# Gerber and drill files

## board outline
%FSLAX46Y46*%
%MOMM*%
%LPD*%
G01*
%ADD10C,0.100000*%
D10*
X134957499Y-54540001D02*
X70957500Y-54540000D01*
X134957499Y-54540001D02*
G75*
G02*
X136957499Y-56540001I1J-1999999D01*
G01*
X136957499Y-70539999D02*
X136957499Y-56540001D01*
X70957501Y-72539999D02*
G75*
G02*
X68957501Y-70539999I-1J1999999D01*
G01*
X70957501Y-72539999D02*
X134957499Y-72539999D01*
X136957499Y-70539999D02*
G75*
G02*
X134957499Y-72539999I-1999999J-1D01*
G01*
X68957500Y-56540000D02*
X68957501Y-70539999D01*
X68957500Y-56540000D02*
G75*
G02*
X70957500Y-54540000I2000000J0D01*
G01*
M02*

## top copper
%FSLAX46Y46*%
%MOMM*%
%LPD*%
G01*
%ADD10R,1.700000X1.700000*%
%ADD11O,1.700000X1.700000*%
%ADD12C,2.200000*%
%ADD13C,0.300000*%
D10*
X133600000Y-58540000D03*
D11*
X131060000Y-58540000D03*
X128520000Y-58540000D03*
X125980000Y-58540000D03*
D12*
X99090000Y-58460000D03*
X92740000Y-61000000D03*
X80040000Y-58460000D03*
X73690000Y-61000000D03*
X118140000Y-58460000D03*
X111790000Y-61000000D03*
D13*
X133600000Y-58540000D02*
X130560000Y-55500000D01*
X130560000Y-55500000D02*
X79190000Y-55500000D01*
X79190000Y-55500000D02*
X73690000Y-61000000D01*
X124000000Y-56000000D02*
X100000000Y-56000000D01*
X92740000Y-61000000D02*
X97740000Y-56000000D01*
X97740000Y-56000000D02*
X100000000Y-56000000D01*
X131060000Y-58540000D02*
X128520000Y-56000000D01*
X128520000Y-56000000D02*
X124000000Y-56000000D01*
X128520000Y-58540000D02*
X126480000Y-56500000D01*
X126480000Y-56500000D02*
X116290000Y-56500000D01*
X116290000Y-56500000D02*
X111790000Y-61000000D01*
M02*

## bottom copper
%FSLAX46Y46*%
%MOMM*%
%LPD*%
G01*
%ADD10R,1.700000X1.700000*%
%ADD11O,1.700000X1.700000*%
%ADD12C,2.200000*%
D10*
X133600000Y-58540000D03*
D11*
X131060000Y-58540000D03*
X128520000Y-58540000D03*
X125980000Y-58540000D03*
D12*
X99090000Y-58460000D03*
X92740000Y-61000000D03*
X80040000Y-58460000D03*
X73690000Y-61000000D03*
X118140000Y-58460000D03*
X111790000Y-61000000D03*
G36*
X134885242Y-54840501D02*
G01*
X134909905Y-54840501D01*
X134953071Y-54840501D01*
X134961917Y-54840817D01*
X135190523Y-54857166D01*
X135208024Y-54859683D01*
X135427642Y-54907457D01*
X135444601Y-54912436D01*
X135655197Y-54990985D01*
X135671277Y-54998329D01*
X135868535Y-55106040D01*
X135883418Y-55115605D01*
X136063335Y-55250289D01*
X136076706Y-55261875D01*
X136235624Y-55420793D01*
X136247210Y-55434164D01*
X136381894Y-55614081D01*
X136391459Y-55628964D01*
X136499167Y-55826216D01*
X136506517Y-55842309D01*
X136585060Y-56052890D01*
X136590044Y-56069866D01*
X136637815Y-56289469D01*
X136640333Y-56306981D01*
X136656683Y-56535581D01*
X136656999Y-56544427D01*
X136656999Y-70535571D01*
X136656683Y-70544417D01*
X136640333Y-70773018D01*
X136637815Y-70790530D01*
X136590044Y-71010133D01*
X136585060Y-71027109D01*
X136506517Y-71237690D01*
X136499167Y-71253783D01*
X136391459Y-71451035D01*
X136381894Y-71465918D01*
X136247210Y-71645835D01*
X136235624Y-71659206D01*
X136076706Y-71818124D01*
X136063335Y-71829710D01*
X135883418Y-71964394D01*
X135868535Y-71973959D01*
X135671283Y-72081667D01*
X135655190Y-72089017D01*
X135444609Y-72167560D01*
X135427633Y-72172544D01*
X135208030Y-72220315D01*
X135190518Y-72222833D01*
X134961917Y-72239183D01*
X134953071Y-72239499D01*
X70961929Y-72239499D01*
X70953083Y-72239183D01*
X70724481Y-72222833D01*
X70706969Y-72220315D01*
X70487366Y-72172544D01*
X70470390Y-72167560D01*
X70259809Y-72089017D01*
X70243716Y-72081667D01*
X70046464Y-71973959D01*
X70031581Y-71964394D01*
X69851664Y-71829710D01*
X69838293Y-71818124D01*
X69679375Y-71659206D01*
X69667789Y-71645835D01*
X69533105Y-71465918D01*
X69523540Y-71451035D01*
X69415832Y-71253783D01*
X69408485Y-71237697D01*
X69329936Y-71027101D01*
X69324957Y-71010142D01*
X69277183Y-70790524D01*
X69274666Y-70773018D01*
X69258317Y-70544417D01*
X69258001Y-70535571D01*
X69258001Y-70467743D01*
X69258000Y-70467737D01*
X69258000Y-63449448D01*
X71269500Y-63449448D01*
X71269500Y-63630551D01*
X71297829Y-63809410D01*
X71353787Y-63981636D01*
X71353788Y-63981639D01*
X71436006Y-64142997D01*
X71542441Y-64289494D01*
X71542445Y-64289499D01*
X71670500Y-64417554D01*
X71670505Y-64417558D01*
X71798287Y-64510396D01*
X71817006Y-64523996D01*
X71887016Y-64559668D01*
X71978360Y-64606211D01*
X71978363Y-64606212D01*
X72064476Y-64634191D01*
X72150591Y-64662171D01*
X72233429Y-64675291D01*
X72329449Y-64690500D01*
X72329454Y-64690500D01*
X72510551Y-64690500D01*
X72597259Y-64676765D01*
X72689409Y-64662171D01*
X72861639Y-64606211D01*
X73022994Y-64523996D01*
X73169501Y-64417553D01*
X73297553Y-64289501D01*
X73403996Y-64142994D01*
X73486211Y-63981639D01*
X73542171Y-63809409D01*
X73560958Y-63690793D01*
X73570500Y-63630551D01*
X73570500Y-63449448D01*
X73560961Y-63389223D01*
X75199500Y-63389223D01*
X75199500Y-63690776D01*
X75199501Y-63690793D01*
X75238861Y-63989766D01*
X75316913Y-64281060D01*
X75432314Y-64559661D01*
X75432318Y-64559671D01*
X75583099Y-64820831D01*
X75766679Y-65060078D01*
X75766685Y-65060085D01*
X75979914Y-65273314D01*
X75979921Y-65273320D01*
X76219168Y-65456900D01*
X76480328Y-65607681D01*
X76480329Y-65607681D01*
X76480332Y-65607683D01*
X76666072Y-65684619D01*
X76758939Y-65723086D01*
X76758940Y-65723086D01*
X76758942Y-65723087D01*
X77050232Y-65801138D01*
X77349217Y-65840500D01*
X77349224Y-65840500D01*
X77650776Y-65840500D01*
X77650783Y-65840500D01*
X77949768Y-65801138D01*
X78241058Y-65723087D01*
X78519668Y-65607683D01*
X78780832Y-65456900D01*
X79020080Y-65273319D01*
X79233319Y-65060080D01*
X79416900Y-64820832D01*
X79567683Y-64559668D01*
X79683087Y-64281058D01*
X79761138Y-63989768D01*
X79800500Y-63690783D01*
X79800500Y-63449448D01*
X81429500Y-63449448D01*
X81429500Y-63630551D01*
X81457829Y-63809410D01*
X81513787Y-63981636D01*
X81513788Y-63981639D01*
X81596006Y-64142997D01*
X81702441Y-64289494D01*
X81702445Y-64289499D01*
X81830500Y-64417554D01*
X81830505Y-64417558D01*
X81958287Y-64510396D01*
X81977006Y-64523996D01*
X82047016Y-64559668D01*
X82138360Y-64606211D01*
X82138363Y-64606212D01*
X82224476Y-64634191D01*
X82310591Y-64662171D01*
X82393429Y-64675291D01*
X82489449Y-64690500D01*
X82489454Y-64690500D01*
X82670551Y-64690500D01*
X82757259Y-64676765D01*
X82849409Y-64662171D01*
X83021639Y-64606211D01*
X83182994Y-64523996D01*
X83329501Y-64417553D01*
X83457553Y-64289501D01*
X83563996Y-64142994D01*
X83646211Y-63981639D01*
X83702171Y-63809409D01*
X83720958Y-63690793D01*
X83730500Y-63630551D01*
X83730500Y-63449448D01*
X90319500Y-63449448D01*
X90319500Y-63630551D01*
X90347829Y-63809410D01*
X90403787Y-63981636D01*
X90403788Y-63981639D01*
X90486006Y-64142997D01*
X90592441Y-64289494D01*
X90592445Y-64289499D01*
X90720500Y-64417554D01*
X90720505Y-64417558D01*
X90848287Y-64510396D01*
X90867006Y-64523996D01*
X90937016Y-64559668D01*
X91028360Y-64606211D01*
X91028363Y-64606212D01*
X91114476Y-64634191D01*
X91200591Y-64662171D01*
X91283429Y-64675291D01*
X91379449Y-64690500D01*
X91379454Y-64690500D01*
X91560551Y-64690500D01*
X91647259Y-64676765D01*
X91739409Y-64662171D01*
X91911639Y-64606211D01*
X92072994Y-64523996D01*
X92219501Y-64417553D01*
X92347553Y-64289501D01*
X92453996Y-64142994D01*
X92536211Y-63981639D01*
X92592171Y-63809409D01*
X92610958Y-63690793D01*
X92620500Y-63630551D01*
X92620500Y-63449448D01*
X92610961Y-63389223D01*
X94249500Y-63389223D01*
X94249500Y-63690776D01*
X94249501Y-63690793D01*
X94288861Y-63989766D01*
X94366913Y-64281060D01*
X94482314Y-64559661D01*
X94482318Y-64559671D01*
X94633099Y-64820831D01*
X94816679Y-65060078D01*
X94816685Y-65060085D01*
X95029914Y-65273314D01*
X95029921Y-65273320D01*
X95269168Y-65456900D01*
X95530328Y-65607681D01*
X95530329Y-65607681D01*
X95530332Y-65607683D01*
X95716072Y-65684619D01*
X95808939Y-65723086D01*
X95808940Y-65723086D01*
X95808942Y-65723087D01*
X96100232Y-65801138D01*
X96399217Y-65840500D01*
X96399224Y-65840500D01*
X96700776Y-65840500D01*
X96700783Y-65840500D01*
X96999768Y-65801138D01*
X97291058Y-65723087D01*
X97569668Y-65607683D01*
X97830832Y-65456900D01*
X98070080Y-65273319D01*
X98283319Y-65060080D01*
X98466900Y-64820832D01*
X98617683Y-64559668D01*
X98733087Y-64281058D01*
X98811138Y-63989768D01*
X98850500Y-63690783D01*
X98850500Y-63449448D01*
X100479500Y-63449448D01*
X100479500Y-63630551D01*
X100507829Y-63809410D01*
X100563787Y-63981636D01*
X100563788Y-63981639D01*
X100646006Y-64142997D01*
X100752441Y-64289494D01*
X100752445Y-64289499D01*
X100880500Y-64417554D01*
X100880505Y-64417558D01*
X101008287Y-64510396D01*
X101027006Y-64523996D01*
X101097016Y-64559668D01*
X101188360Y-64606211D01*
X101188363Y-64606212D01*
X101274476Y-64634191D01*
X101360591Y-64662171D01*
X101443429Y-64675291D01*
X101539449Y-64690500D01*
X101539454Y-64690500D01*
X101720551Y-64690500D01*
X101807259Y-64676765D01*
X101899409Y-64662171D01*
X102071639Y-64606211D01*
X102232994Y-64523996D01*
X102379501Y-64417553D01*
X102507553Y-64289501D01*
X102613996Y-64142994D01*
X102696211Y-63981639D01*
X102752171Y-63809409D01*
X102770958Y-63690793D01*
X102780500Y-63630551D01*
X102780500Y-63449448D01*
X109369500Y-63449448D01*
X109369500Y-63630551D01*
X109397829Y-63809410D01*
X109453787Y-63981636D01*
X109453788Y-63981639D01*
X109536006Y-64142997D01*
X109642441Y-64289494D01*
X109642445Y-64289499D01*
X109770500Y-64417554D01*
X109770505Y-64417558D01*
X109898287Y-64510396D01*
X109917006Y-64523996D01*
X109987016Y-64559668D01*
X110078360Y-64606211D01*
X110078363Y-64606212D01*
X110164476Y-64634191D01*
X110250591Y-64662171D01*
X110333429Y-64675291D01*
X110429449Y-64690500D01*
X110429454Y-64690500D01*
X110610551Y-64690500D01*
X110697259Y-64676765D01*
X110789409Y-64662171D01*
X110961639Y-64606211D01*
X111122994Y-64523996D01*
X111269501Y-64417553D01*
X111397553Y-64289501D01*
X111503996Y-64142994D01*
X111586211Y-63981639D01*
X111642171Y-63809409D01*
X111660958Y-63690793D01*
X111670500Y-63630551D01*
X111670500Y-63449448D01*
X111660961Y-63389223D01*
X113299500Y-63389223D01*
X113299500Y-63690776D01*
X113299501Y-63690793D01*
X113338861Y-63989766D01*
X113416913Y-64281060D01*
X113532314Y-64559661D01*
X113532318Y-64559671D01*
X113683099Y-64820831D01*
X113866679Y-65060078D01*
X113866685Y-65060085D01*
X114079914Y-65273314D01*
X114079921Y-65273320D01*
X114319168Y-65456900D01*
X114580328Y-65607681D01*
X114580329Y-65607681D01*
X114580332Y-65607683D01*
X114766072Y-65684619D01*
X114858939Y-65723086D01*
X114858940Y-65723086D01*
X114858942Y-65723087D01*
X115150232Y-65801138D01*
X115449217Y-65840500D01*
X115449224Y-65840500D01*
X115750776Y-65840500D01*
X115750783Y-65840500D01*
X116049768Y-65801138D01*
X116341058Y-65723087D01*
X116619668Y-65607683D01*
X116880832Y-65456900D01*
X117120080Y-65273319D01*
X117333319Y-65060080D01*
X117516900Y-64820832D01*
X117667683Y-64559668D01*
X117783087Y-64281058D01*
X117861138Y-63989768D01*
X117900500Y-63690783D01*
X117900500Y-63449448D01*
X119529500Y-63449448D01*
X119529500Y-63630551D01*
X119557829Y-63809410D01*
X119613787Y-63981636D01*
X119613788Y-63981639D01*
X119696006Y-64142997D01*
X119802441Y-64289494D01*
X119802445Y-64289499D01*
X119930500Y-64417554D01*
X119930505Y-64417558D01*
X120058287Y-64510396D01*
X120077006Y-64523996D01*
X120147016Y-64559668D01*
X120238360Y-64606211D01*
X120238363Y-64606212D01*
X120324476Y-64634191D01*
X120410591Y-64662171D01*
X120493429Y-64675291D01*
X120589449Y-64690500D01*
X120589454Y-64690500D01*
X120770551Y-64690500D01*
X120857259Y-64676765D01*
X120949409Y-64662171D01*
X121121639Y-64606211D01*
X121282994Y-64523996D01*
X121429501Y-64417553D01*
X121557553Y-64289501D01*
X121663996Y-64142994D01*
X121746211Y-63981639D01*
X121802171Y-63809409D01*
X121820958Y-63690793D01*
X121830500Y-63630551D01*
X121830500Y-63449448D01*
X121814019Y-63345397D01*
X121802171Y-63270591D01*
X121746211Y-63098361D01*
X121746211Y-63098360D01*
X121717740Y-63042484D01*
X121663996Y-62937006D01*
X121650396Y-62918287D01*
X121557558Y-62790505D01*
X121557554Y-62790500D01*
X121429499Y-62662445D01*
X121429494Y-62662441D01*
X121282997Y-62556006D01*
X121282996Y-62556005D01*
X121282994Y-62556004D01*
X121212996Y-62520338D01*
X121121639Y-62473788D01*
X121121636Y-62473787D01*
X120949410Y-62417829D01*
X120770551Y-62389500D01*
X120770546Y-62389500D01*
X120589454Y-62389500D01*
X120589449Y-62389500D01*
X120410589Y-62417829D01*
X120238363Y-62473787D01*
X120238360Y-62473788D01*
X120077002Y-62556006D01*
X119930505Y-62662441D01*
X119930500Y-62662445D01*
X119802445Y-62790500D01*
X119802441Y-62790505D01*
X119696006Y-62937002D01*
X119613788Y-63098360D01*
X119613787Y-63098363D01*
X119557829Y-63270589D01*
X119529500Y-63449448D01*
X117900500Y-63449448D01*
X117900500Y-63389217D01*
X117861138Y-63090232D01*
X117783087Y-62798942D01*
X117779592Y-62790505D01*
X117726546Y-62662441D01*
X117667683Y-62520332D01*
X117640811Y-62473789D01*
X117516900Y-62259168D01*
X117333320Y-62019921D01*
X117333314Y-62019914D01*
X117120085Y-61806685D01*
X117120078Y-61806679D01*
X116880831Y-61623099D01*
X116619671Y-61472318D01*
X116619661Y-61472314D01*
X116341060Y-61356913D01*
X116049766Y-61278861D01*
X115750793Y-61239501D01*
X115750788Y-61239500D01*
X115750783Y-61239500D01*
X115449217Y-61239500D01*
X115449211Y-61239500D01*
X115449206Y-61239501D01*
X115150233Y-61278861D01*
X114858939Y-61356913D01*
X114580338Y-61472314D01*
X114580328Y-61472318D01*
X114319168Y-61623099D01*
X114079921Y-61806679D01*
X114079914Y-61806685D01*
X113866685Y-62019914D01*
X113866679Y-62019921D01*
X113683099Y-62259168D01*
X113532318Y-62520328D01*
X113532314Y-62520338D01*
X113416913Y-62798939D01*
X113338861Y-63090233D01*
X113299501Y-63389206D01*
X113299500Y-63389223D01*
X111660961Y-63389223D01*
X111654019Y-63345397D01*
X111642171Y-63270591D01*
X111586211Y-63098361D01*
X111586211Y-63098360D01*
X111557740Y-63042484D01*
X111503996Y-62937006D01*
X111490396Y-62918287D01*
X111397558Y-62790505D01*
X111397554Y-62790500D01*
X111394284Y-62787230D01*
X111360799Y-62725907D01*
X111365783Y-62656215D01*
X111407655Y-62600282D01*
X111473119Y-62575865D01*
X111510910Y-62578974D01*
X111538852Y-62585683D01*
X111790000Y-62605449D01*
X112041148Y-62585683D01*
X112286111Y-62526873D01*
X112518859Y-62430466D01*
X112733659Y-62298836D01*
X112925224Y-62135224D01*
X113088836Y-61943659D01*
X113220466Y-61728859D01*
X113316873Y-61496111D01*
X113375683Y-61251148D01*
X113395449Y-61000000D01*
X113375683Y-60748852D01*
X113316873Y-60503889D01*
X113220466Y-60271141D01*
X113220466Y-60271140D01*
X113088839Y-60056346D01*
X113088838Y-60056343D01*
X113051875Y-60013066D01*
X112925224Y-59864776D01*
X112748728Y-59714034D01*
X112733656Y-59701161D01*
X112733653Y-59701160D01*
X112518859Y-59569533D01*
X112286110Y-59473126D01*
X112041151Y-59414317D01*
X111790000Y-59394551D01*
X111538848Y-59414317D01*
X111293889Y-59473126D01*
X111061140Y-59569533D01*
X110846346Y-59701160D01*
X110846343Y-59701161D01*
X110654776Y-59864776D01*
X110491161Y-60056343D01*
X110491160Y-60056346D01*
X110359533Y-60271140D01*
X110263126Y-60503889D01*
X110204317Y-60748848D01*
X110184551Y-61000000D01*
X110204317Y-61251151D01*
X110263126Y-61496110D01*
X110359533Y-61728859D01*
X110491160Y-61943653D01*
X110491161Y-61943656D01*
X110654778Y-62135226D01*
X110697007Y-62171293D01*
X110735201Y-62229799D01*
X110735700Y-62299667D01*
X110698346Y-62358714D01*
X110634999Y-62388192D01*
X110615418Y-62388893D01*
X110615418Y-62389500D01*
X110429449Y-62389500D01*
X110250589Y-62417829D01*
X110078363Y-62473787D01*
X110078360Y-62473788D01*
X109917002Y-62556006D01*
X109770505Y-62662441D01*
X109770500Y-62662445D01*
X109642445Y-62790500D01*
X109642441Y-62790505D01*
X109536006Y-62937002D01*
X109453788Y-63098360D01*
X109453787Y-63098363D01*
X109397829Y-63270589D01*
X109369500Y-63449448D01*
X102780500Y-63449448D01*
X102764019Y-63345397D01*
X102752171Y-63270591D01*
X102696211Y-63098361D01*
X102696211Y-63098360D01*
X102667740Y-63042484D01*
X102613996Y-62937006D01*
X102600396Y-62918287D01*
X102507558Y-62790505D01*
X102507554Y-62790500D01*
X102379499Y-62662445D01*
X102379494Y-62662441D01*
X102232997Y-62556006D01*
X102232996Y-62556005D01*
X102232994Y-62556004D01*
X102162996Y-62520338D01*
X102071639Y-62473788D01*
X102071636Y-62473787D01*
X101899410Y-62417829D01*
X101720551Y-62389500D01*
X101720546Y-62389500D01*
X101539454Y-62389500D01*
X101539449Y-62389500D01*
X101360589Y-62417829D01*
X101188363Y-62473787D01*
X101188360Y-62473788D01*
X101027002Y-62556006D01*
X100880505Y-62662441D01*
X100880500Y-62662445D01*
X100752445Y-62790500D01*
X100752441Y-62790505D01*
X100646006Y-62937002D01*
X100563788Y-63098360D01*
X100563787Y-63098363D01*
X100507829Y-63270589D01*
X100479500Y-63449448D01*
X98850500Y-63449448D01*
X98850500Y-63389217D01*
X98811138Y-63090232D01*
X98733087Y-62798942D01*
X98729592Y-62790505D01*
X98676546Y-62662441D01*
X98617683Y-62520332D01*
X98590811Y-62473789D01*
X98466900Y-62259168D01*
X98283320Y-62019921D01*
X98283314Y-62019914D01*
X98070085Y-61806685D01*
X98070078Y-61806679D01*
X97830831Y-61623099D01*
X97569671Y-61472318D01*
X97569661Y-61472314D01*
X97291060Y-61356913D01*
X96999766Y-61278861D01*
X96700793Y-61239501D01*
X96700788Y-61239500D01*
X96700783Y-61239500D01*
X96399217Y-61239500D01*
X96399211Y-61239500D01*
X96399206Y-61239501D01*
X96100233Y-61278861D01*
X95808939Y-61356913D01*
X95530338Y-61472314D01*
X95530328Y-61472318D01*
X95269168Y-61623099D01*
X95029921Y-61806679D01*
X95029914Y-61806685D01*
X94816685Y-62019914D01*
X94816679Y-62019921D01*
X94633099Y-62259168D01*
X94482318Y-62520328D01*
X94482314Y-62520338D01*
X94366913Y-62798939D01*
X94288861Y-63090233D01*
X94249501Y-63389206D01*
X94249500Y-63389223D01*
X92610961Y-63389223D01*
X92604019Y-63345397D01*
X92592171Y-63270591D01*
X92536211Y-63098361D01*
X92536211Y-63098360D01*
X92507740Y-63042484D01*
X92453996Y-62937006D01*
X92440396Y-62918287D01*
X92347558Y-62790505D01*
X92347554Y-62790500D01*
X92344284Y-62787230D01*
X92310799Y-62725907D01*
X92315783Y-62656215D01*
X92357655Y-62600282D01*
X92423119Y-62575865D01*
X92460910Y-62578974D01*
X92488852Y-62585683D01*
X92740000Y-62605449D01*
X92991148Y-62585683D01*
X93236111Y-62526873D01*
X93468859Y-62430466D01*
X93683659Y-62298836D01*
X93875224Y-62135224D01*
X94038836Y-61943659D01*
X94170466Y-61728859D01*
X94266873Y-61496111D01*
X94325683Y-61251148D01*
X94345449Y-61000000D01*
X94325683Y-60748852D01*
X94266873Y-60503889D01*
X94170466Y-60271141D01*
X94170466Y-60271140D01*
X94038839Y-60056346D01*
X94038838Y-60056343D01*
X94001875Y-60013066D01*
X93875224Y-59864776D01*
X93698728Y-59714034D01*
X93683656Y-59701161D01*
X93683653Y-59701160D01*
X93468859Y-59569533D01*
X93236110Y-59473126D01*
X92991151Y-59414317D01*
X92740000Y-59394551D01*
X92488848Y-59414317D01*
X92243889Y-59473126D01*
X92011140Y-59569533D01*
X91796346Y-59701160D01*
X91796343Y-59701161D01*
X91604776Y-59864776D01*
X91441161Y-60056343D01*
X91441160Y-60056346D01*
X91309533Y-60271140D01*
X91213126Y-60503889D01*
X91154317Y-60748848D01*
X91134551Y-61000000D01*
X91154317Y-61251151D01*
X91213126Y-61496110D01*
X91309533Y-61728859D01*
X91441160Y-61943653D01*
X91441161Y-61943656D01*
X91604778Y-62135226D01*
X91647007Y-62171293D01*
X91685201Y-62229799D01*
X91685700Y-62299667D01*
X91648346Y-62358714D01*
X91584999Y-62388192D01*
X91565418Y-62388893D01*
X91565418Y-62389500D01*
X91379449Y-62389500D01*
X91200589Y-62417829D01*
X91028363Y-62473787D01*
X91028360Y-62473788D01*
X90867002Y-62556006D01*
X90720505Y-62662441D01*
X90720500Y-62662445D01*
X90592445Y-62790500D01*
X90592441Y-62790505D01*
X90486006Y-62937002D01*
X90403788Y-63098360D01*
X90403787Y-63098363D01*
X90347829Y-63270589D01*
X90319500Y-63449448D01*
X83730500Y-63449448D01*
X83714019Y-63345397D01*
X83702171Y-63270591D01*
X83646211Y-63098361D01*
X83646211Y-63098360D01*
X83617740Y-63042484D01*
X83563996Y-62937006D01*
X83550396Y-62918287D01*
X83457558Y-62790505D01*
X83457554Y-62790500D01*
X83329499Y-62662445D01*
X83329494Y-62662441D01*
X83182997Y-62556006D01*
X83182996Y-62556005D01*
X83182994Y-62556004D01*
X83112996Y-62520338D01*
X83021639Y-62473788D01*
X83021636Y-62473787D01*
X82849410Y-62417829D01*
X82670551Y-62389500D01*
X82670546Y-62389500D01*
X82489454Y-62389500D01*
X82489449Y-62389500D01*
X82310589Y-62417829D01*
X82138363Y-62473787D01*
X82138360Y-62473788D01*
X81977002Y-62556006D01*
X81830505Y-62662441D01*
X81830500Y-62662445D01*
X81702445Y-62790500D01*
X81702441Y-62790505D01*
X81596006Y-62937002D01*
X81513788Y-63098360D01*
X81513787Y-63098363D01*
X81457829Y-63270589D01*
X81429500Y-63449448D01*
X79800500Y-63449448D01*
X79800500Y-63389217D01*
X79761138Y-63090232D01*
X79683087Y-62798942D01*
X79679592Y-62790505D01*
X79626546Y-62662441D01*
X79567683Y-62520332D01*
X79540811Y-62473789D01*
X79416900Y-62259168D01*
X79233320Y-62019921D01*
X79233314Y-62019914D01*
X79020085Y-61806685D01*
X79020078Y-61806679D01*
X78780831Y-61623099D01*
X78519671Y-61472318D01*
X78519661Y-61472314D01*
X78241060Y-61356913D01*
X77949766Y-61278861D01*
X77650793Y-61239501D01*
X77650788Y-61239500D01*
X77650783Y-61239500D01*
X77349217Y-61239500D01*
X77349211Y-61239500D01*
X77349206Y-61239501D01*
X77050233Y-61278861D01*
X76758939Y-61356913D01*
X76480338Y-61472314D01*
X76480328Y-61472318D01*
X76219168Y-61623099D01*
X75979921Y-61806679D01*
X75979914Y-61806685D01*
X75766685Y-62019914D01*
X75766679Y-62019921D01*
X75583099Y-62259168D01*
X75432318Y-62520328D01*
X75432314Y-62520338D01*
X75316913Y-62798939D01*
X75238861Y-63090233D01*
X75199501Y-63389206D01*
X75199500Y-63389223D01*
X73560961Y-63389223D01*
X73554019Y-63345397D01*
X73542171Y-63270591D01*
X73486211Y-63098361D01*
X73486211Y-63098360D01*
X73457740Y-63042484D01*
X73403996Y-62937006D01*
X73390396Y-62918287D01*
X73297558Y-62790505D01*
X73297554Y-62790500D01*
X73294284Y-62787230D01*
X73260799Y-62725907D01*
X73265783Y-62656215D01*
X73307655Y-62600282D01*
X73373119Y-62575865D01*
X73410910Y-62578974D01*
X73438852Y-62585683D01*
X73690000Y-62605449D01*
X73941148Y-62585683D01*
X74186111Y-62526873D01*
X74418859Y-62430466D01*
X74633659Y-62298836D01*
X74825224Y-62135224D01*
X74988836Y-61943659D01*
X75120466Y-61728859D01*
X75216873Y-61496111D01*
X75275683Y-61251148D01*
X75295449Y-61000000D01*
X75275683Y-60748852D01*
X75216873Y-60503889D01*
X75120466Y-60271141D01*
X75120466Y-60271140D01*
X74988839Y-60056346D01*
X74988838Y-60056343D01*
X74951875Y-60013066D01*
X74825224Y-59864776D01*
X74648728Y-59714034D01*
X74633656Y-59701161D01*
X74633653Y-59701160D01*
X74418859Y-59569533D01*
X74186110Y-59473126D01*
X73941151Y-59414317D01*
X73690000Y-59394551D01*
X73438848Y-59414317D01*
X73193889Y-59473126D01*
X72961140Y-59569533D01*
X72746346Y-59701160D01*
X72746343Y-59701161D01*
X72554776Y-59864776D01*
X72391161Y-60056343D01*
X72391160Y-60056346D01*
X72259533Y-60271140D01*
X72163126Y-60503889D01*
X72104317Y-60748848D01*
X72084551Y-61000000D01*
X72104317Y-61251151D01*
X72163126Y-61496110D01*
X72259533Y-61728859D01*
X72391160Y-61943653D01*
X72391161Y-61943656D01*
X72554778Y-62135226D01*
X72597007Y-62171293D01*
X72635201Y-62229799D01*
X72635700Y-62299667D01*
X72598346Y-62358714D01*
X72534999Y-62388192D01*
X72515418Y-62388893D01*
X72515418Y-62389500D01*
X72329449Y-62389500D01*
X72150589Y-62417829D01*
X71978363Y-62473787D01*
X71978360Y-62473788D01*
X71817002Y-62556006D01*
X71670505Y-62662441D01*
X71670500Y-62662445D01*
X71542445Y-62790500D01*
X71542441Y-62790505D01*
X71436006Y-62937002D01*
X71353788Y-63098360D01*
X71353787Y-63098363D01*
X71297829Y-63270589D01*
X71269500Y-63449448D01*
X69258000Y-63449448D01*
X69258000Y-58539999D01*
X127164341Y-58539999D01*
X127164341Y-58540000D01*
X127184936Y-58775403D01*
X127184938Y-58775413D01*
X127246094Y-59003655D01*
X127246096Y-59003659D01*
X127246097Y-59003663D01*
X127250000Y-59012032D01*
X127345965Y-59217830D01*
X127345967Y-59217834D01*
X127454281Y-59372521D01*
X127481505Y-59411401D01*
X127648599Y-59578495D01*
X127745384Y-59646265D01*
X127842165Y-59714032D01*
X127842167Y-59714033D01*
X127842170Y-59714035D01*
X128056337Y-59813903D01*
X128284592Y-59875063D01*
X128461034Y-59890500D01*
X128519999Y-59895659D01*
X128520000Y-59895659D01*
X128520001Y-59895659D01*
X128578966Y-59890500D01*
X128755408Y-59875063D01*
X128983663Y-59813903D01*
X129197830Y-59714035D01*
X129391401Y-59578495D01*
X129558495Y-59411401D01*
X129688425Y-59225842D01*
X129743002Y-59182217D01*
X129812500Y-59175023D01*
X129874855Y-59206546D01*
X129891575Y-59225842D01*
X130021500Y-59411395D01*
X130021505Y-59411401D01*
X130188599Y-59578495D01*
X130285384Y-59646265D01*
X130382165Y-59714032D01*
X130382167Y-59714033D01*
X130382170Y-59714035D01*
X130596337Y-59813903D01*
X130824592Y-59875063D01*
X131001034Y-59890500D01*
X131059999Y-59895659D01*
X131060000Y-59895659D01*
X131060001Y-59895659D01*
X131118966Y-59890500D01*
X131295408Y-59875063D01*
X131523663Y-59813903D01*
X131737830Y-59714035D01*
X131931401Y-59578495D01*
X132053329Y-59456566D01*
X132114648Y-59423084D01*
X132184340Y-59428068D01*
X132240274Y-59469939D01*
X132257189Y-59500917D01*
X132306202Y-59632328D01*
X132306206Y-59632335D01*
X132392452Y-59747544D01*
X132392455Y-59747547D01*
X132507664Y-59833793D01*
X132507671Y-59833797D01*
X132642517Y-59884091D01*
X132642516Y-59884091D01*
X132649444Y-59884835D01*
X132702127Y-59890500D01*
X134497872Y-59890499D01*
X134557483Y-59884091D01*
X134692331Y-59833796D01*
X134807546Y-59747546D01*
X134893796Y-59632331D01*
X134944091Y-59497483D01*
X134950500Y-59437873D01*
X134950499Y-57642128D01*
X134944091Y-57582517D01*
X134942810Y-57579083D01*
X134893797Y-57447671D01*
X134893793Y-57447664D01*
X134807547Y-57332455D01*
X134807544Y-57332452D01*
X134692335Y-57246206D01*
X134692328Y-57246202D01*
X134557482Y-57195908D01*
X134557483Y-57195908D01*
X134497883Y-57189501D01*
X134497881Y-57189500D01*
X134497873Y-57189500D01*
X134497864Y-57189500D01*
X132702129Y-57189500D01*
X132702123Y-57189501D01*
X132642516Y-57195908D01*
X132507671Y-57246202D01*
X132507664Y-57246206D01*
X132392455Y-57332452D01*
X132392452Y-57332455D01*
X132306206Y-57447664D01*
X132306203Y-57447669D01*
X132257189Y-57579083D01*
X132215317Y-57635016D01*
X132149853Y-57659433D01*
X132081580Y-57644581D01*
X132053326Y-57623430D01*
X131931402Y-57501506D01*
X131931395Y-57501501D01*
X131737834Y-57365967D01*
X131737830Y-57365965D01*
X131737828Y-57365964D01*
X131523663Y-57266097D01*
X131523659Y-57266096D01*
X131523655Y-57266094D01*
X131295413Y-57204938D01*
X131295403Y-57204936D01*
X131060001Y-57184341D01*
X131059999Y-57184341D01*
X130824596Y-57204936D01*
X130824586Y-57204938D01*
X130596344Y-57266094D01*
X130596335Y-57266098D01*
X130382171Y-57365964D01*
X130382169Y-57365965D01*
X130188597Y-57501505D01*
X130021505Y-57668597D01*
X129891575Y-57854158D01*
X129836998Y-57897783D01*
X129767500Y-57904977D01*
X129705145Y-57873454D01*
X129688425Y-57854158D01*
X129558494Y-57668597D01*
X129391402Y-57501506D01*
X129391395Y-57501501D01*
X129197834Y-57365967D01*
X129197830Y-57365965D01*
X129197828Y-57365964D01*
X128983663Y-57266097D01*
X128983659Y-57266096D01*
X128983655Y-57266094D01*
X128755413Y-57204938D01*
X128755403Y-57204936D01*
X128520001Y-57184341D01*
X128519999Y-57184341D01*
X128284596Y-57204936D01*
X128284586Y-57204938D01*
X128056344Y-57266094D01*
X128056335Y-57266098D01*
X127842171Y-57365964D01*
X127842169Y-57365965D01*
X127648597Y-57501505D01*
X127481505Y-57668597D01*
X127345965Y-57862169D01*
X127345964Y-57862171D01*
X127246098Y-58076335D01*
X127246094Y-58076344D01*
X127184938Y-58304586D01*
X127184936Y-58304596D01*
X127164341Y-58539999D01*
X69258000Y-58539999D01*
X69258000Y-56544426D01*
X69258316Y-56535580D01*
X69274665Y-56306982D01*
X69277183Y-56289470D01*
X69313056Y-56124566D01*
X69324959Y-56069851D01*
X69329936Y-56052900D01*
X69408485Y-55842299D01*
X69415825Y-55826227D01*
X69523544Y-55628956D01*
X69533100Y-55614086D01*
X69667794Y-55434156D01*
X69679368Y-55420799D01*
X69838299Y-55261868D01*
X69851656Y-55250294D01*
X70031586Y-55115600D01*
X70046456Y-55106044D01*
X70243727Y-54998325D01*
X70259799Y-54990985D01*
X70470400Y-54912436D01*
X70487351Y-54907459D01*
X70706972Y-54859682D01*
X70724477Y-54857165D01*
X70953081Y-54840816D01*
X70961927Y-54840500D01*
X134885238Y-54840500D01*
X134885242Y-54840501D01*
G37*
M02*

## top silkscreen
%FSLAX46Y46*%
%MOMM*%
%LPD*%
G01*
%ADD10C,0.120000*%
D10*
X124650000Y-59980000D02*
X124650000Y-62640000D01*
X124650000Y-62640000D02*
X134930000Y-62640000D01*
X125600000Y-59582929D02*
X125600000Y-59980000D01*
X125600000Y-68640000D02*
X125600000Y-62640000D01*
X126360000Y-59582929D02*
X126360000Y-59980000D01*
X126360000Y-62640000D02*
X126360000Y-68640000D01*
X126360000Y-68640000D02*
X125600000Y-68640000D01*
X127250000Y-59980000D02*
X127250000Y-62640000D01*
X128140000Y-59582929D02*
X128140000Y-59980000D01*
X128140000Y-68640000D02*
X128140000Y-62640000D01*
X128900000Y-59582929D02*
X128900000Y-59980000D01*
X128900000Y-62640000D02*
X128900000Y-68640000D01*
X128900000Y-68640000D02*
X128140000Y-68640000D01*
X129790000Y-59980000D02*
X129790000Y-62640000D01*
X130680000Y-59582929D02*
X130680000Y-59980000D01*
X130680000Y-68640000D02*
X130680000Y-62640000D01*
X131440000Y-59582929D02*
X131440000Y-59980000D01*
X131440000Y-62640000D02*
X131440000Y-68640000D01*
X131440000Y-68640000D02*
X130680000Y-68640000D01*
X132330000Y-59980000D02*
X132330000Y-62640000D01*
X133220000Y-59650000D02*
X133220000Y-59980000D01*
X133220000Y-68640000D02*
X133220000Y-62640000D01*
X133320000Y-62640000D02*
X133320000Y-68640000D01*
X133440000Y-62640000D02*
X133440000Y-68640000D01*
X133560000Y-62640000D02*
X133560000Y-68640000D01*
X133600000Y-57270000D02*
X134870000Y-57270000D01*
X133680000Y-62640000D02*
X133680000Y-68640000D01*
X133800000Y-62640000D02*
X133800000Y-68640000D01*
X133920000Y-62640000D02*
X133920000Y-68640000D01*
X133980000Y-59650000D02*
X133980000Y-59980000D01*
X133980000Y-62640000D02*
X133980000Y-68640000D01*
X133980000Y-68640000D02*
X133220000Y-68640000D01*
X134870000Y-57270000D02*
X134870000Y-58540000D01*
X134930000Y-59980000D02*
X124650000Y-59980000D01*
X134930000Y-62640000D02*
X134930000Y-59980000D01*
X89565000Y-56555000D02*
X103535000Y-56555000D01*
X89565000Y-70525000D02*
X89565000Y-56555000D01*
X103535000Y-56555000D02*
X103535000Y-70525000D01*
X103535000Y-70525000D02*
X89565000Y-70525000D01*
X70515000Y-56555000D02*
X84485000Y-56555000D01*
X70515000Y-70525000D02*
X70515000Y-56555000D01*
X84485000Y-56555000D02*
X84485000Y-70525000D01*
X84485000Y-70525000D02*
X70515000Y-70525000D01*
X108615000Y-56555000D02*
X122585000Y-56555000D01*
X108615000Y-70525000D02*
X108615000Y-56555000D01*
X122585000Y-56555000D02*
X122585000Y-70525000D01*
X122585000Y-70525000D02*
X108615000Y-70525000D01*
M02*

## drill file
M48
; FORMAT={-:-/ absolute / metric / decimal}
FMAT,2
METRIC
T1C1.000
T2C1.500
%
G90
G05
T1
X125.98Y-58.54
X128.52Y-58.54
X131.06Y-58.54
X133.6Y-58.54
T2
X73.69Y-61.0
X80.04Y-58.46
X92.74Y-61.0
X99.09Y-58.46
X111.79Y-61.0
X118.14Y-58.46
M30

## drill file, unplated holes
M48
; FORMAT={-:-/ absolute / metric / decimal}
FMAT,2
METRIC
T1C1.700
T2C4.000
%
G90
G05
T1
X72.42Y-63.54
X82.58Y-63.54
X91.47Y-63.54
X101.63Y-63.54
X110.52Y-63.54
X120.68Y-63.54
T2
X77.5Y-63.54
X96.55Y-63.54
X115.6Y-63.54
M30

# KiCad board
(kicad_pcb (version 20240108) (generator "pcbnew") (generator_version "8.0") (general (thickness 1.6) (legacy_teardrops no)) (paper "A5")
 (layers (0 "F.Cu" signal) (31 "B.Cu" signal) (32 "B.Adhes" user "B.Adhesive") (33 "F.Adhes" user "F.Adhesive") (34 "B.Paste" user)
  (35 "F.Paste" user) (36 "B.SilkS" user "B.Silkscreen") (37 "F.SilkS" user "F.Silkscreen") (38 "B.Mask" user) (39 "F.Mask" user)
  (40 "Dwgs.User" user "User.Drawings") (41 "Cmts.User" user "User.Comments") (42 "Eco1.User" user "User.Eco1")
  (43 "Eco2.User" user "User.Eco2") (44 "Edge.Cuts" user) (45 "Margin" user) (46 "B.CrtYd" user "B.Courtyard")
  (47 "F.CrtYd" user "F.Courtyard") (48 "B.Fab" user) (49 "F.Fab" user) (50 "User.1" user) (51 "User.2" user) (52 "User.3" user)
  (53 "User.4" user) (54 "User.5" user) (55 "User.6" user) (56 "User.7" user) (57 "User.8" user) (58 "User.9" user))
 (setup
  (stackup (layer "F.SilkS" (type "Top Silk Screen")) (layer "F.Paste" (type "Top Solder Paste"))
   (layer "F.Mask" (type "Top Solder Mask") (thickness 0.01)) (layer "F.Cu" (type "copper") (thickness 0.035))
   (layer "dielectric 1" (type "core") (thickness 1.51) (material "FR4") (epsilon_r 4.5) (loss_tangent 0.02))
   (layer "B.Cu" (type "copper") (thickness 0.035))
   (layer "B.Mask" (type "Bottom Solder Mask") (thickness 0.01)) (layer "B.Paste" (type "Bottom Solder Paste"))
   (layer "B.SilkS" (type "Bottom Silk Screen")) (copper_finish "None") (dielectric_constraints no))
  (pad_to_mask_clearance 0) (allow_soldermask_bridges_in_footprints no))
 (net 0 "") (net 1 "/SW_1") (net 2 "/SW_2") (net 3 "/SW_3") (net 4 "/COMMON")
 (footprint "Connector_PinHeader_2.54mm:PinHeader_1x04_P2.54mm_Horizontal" (layer "F.Cu") (at 133.6 58.54 -90)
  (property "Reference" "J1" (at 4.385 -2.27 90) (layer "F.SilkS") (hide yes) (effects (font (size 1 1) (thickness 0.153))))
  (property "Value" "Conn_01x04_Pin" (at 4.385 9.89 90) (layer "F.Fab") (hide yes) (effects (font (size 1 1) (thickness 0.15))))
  (fp_line (start 1.44 8.95) (end 4.1 8.95) (stroke (width 0.12) (type solid)) (layer "F.SilkS"))
  (fp_line (start 4.1 8.95) (end 4.1 -1.33) (stroke (width 0.12) (type solid)) (layer "F.SilkS"))
  (fp_line (start 1.042929 8) (end 1.44 8) (stroke (width 0.12) (type solid)) (layer "F.SilkS"))
  (fp_line (start 10.1 8) (end 4.1 8) (stroke (width 0.12) (type solid)) (layer "F.SilkS"))
  (fp_line (start 1.042929 7.24) (end 1.44 7.24) (stroke (width 0.12) (type solid)) (layer "F.SilkS"))
  (fp_line (start 4.1 7.24) (end 10.1 7.24) (stroke (width 0.12) (type solid)) (layer "F.SilkS"))
  (fp_line (start 10.1 7.24) (end 10.1 8) (stroke (width 0.12) (type solid)) (layer "F.SilkS"))
  (fp_line (start 1.44 6.35) (end 4.1 6.35) (stroke (width 0.12) (type solid)) (layer "F.SilkS"))
  (fp_line (start 1.042929 5.46) (end 1.44 5.46) (stroke (width 0.12) (type solid)) (layer "F.SilkS"))
  (fp_line (start 10.1 5.46) (end 4.1 5.46) (stroke (width 0.12) (type solid)) (layer "F.SilkS"))
  (fp_line (start 1.042929 4.7) (end 1.44 4.7) (stroke (width 0.12) (type solid)) (layer "F.SilkS"))
  (fp_line (start 4.1 4.7) (end 10.1 4.7) (stroke (width 0.12) (type solid)) (layer "F.SilkS"))
  (fp_line (start 10.1 4.7) (end 10.1 5.46) (stroke (width 0.12) (type solid)) (layer "F.SilkS"))
  (fp_line (start 1.44 3.81) (end 4.1 3.81) (stroke (width 0.12) (type solid)) (layer "F.SilkS"))
  (fp_line (start 1.042929 2.92) (end 1.44 2.92) (stroke (width 0.12) (type solid)) (layer "F.SilkS"))
  (fp_line (start 10.1 2.92) (end 4.1 2.92) (stroke (width 0.12) (type solid)) (layer "F.SilkS"))
  (fp_line (start 1.042929 2.16) (end 1.44 2.16) (stroke (width 0.12) (type solid)) (layer "F.SilkS"))
  (fp_line (start 4.1 2.16) (end 10.1 2.16) (stroke (width 0.12) (type solid)) (layer "F.SilkS"))
  (fp_line (start 10.1 2.16) (end 10.1 2.92) (stroke (width 0.12) (type solid)) (layer "F.SilkS"))
  (fp_line (start 1.44 1.27) (end 4.1 1.27) (stroke (width 0.12) (type solid)) (layer "F.SilkS"))
  (fp_line (start 1.11 0.38) (end 1.44 0.38) (stroke (width 0.12) (type solid)) (layer "F.SilkS"))
  (fp_line (start 10.1 0.38) (end 4.1 0.38) (stroke (width 0.12) (type solid)) (layer "F.SilkS"))
  (fp_line (start 4.1 0.28) (end 10.1 0.28) (stroke (width 0.12) (type solid)) (layer "F.SilkS"))
  (fp_line (start 4.1 0.16) (end 10.1 0.16) (stroke (width 0.12) (type solid)) (layer "F.SilkS"))
  (fp_line (start 4.1 0.04) (end 10.1 0.04) (stroke (width 0.12) (type solid)) (layer "F.SilkS"))
  (fp_line (start -1.27 0) (end -1.27 -1.27) (stroke (width 0.12) (type solid)) (layer "F.SilkS"))
  (fp_line (start 4.1 -0.08) (end 10.1 -0.08) (stroke (width 0.12) (type solid)) (layer "F.SilkS"))
  (fp_line (start 4.1 -0.2) (end 10.1 -0.2) (stroke (width 0.12) (type solid)) (layer "F.SilkS"))
  (fp_line (start 4.1 -0.32) (end 10.1 -0.32) (stroke (width 0.12) (type solid)) (layer "F.SilkS"))
  (fp_line (start 1.11 -0.38) (end 1.44 -0.38) (stroke (width 0.12) (type solid)) (layer "F.SilkS"))
  (fp_line (start 4.1 -0.38) (end 10.1 -0.38) (stroke (width 0.12) (type solid)) (layer "F.SilkS"))
  (fp_line (start 10.1 -0.38) (end 10.1 0.38) (stroke (width 0.12) (type solid)) (layer "F.SilkS"))
  (fp_line (start -1.27 -1.27) (end 0 -1.27) (stroke (width 0.12) (type solid)) (layer "F.SilkS"))
  (fp_line (start 1.44 -1.33) (end 1.44 8.95) (stroke (width 0.12) (type solid)) (layer "F.SilkS"))
  (fp_line (start 4.1 -1.33) (end 1.44 -1.33) (stroke (width 0.12) (type solid)) (layer "F.SilkS"))
  (pad "1" thru_hole rect (at 0 0 270) (size 1.7 1.7) (drill 1) (layers "*.Cu" "*.Mask") (remove_unused_layers no) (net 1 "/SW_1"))
  (pad "2" thru_hole oval (at 0 2.54 270) (size 1.7 1.7) (drill 1) (layers "*.Cu" "*.Mask") (remove_unused_layers no) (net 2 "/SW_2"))
  (pad "3" thru_hole oval (at 0 5.08 270) (size 1.7 1.7) (drill 1) (layers "*.Cu" "*.Mask") (remove_unused_layers no) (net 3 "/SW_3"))
  (pad "4" thru_hole oval (at 0 7.62 270) (size 1.7 1.7) (drill 1) (layers "*.Cu" "*.Mask") (remove_unused_layers no) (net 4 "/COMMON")))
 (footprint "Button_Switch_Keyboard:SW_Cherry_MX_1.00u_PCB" (layer "F.Cu") (at 99.09 58.46)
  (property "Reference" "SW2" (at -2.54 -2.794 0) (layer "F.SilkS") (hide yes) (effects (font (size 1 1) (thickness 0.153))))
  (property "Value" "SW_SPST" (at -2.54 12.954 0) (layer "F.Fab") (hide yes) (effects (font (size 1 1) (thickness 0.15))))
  (fp_line (start -9.525 -1.905) (end 4.445 -1.905) (stroke (width 0.12) (type solid)) (layer "F.SilkS"))
  (fp_line (start -9.525 12.065) (end -9.525 -1.905) (stroke (width 0.12) (type solid)) (layer "F.SilkS"))
  (fp_line (start 4.445 -1.905) (end 4.445 12.065) (stroke (width 0.12) (type solid)) (layer "F.SilkS"))
  (fp_line (start 4.445 12.065) (end -9.525 12.065) (stroke (width 0.12) (type solid)) (layer "F.SilkS"))
  (pad "" np_thru_hole circle (at -7.62 5.08) (size 1.7 1.7) (drill 1.7) (layers "*.Cu" "*.Mask"))
  (pad "" np_thru_hole circle (at -2.54 5.08) (size 4 4) (drill 4) (layers "*.Cu" "*.Mask"))
  (pad "" np_thru_hole circle (at 2.54 5.08) (size 1.7 1.7) (drill 1.7) (layers "*.Cu" "*.Mask"))
  (pad "1" thru_hole circle (at 0 0) (size 2.2 2.2) (drill 1.5) (layers "*.Cu" "*.Mask") (remove_unused_layers no) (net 4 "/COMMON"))
  (pad "2" thru_hole circle (at -6.35 2.54) (size 2.2 2.2) (drill 1.5) (layers "*.Cu" "*.Mask") (remove_unused_layers no) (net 2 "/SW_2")))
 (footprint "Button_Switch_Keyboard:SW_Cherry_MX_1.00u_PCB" (layer "F.Cu") (at 80.04 58.46)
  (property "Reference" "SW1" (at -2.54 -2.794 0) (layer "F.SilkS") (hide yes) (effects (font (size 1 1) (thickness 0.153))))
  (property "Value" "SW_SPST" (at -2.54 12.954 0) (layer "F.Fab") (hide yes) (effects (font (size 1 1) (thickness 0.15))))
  (fp_line (start -9.525 -1.905) (end 4.445 -1.905) (stroke (width 0.12) (type solid)) (layer "F.SilkS"))
  (fp_line (start -9.525 12.065) (end -9.525 -1.905) (stroke (width 0.12) (type solid)) (layer "F.SilkS"))
  (fp_line (start 4.445 -1.905) (end 4.445 12.065) (stroke (width 0.12) (type solid)) (layer "F.SilkS"))
  (fp_line (start 4.445 12.065) (end -9.525 12.065) (stroke (width 0.12) (type solid)) (layer "F.SilkS"))
  (pad "" np_thru_hole circle (at -7.62 5.08) (size 1.7 1.7) (drill 1.7) (layers "*.Cu" "*.Mask"))
  (pad "" np_thru_hole circle (at -2.54 5.08) (size 4 4) (drill 4) (layers "*.Cu" "*.Mask"))
  (pad "" np_thru_hole circle (at 2.54 5.08) (size 1.7 1.7) (drill 1.7) (layers "*.Cu" "*.Mask"))
  (pad "1" thru_hole circle (at 0 0) (size 2.2 2.2) (drill 1.5) (layers "*.Cu" "*.Mask") (remove_unused_layers no) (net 4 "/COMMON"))
  (pad "2" thru_hole circle (at -6.35 2.54) (size 2.2 2.2) (drill 1.5) (layers "*.Cu" "*.Mask") (remove_unused_layers no) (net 1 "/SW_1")))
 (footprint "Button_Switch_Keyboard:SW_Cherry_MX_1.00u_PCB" (layer "F.Cu") (at 118.14 58.46)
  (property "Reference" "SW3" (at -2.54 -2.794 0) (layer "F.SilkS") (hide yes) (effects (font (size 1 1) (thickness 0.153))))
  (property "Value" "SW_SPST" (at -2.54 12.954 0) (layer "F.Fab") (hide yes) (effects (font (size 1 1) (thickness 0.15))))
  (fp_line (start -9.525 -1.905) (end 4.445 -1.905) (stroke (width 0.12) (type solid)) (layer "F.SilkS"))
  (fp_line (start -9.525 12.065) (end -9.525 -1.905) (stroke (width 0.12) (type solid)) (layer "F.SilkS"))
  (fp_line (start 4.445 -1.905) (end 4.445 12.065) (stroke (width 0.12) (type solid)) (layer "F.SilkS"))
  (fp_line (start 4.445 12.065) (end -9.525 12.065) (stroke (width 0.12) (type solid)) (layer "F.SilkS"))
  (pad "" np_thru_hole circle (at -7.62 5.08) (size 1.7 1.7) (drill 1.7) (layers "*.Cu" "*.Mask"))
  (pad "" np_thru_hole circle (at -2.54 5.08) (size 4 4) (drill 4) (layers "*.Cu" "*.Mask"))
  (pad "" np_thru_hole circle (at 2.54 5.08) (size 1.7 1.7) (drill 1.7) (layers "*.Cu" "*.Mask"))
  (pad "1" thru_hole circle (at 0 0) (size 2.2 2.2) (drill 1.5) (layers "*.Cu" "*.Mask") (remove_unused_layers no) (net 4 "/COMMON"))
  (pad "2" thru_hole circle (at -6.35 2.54) (size 2.2 2.2) (drill 1.5) (layers "*.Cu" "*.Mask") (remove_unused_layers no) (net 3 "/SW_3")))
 (gr_line (start 134.957499 54.540001) (end 70.9575 54.54) (stroke (width 0.1) (type default)) (layer "Edge.Cuts"))
 (gr_arc (start 134.957499 54.540001) (mid 136.371713 55.125787) (end 136.957499 56.540001) (stroke (width 0.1) (type default))
  (layer "Edge.Cuts"))
 (gr_line (start 136.957499 70.539999) (end 136.957499 56.540001) (stroke (width 0.1) (type default)) (layer "Edge.Cuts"))
 (gr_arc (start 70.957501 72.539999) (mid 69.543287 71.954213) (end 68.957501 70.539999) (stroke (width 0.1) (type default))
  (layer "Edge.Cuts"))
 (gr_line (start 70.957501 72.539999) (end 134.957499 72.539999) (stroke (width 0.1) (type default)) (layer "Edge.Cuts"))
 (gr_arc (start 136.957499 70.539999) (mid 136.371713 71.954213) (end 134.957499 72.539999) (stroke (width 0.1) (type default))
  (layer "Edge.Cuts"))
 (gr_line (start 68.9575 56.54) (end 68.957501 70.539999) (stroke (width 0.1) (type default)) (layer "Edge.Cuts"))
 (gr_arc (start 68.9575 56.54) (mid 69.543286 55.125786) (end 70.9575 54.54) (stroke (width 0.1) (type default)) (layer "Edge.Cuts"))
 (segment (start 79.19 55.5) (end 73.69 61) (width 0.3) (layer "F.Cu") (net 1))
 (segment (start 130.56 55.5) (end 79.19 55.5) (width 0.3) (layer "F.Cu") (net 1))
 (segment (start 133.6 58.54) (end 130.56 55.5) (width 0.3) (layer "F.Cu") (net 1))
 (segment (start 126.48 56.5) (end 116.29 56.5) (width 0.3) (layer "F.Cu") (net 3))
 (segment (start 116.29 56.5) (end 111.79 61) (width 0.3) (layer "F.Cu") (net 3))
 (segment (start 128.52 58.54) (end 126.48 56.5) (width 0.3) (layer "F.Cu") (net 3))
 (segment (start 124 56) (end 100 56) (width 0.3) (layer "F.Cu") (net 2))
 (segment (start 128.52 56) (end 124 56) (width 0.3) (layer "F.Cu") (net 2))
 (segment (start 92.74 61) (end 97.74 56) (width 0.3) (layer "F.Cu") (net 2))
 (segment (start 131.06 58.54) (end 128.52 56) (width 0.3) (layer "F.Cu") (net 2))
 (segment (start 97.74 56) (end 100 56) (width 0.3) (layer "F.Cu") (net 2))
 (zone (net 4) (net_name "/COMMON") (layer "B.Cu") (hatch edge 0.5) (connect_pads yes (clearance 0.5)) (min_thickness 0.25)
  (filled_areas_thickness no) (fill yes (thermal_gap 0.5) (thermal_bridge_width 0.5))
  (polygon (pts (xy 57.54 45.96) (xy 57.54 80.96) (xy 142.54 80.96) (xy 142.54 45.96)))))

